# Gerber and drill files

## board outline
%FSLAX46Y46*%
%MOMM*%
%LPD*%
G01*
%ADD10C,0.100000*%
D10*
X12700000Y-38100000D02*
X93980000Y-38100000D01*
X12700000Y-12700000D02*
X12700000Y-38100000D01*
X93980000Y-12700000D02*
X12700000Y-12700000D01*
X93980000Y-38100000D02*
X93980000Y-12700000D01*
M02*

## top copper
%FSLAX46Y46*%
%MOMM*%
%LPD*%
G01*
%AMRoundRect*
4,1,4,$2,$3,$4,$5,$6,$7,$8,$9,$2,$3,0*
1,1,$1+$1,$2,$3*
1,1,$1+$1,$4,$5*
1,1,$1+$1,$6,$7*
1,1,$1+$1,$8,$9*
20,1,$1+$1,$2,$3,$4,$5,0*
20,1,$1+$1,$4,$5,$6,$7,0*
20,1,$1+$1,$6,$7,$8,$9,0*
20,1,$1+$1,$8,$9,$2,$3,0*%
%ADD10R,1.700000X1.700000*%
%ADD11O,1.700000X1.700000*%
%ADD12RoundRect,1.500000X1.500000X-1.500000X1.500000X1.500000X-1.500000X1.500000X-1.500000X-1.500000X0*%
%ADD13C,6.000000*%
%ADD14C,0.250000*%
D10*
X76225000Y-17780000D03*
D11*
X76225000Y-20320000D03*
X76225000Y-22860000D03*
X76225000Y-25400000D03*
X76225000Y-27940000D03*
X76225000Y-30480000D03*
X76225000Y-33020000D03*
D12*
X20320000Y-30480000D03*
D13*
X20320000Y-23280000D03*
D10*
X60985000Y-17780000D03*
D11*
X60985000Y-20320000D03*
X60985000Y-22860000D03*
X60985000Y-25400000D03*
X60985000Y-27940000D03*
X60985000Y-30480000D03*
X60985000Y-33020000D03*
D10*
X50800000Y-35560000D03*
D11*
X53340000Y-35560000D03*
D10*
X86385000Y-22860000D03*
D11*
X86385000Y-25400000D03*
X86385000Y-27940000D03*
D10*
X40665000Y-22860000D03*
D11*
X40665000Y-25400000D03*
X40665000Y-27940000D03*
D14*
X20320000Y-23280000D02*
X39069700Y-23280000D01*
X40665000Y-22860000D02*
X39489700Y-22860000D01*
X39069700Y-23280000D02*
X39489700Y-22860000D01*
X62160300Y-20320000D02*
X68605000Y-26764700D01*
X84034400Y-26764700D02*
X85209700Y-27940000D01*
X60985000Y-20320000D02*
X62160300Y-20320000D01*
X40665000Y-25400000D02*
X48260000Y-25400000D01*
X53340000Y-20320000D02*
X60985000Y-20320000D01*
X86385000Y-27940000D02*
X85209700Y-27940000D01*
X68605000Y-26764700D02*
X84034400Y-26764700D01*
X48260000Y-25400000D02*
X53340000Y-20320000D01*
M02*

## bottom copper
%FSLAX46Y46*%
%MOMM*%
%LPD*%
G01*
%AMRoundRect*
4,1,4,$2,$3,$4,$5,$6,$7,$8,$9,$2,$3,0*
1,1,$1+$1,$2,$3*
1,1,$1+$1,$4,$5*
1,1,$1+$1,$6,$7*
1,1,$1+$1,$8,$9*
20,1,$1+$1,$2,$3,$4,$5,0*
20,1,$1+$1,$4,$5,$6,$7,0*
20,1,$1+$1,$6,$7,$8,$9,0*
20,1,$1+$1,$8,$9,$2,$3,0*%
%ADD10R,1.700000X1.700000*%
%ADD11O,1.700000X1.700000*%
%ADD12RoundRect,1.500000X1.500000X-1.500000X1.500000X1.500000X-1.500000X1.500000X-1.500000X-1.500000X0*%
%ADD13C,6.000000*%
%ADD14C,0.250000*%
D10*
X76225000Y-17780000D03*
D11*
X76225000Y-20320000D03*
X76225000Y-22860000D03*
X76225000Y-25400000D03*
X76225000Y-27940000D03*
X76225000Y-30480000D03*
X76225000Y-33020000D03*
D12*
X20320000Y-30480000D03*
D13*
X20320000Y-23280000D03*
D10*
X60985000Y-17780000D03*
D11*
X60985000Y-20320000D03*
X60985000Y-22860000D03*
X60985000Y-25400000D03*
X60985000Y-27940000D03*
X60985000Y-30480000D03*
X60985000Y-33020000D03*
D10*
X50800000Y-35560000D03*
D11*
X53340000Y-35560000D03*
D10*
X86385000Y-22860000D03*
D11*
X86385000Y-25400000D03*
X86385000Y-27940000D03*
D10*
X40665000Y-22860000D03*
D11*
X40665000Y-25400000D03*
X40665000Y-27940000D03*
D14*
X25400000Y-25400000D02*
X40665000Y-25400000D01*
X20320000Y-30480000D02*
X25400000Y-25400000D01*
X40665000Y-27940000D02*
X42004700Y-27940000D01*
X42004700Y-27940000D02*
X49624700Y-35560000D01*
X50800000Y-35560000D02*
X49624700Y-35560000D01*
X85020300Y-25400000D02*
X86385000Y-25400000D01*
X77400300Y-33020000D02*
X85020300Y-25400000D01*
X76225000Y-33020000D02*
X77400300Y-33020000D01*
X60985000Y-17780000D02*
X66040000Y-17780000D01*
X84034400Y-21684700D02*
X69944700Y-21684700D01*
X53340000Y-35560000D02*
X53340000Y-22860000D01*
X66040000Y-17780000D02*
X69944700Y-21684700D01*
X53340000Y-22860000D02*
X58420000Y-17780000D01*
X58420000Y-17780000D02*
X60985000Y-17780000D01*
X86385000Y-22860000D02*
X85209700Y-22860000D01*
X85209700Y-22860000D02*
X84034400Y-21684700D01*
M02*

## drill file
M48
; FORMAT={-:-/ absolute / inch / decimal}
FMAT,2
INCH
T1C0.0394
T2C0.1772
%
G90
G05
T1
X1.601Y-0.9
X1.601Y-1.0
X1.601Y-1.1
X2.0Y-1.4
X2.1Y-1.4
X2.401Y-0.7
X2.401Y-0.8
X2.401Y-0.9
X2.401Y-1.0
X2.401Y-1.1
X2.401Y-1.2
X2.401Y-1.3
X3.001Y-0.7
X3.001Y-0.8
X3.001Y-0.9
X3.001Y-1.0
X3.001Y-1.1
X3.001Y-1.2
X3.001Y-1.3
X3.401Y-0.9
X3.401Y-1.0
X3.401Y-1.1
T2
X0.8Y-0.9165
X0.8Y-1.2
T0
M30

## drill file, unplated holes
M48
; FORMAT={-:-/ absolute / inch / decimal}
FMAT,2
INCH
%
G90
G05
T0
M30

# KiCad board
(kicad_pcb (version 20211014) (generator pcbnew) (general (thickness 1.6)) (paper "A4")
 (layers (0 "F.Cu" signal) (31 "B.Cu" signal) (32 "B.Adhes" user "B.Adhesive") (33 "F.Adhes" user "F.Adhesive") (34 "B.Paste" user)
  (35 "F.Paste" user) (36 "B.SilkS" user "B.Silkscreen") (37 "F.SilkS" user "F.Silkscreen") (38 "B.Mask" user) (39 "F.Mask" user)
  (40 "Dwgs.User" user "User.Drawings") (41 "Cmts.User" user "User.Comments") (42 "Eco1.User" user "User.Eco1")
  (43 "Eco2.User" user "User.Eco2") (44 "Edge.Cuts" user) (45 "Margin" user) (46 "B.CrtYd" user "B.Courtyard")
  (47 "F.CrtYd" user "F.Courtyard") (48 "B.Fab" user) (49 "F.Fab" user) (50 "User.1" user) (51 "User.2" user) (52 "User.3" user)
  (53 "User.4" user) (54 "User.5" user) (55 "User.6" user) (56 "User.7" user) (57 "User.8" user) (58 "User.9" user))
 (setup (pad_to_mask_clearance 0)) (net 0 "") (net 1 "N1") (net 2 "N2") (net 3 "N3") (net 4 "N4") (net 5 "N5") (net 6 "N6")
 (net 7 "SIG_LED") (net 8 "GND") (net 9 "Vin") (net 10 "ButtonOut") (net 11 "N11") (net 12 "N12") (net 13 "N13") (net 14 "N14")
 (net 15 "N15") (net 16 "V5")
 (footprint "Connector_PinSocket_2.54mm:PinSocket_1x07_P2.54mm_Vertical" (layer "F.Cu") (at 76.225 17.78)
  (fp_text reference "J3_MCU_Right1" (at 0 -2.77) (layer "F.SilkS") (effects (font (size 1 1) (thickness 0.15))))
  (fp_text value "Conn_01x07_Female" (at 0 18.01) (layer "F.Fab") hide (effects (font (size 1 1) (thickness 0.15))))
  (pad "1" thru_hole rect (at 0 0) (size 1.7 1.7) (drill 1) (layers *.Cu *.Mask) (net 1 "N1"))
  (pad "2" thru_hole oval (at 0 2.54) (size 1.7 1.7) (drill 1) (layers *.Cu *.Mask) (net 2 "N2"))
  (pad "3" thru_hole oval (at 0 5.08) (size 1.7 1.7) (drill 1) (layers *.Cu *.Mask) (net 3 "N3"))
  (pad "4" thru_hole oval (at 0 7.62) (size 1.7 1.7) (drill 1) (layers *.Cu *.Mask) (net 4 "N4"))
  (pad "5" thru_hole oval (at 0 10.16) (size 1.7 1.7) (drill 1) (layers *.Cu *.Mask) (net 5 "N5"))
  (pad "6" thru_hole oval (at 0 12.7) (size 1.7 1.7) (drill 1) (layers *.Cu *.Mask) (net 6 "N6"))
  (pad "7" thru_hole oval (at 0 15.24) (size 1.7 1.7) (drill 1) (layers *.Cu *.Mask) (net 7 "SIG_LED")))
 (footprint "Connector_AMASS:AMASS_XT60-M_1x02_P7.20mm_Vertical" (layer "F.Cu") (at 20.32 30.48 90)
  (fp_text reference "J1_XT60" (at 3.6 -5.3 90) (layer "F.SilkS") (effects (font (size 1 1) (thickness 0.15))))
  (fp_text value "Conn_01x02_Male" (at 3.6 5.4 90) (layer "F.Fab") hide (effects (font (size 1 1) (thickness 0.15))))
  (pad "1" thru_hole roundrect (at 0 0 90) (size 6 6) (drill 4.5) (layers *.Cu *.Mask) (roundrect_rratio 0.25) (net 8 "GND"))
  (pad "2" thru_hole circle (at 7.2 0 90) (size 6 6) (drill 4.5) (layers *.Cu *.Mask) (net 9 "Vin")))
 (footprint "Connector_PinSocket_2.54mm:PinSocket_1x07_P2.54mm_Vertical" (layer "F.Cu") (at 60.985 17.78)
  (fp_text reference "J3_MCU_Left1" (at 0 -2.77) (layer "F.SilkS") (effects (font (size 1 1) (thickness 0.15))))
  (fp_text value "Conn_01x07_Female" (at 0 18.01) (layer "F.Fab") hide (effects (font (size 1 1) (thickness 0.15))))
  (pad "1" thru_hole rect (at 0 0) (size 1.7 1.7) (drill 1) (layers *.Cu *.Mask) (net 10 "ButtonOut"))
  (pad "2" thru_hole oval (at 0 2.54) (size 1.7 1.7) (drill 1) (layers *.Cu *.Mask) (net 8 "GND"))
  (pad "3" thru_hole oval (at 0 5.08) (size 1.7 1.7) (drill 1) (layers *.Cu *.Mask) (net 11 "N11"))
  (pad "4" thru_hole oval (at 0 7.62) (size 1.7 1.7) (drill 1) (layers *.Cu *.Mask) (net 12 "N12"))
  (pad "5" thru_hole oval (at 0 10.16) (size 1.7 1.7) (drill 1) (layers *.Cu *.Mask) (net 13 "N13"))
  (pad "6" thru_hole oval (at 0 12.7) (size 1.7 1.7) (drill 1) (layers *.Cu *.Mask) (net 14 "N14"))
  (pad "7" thru_hole oval (at 0 15.24) (size 1.7 1.7) (drill 1) (layers *.Cu *.Mask) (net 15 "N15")))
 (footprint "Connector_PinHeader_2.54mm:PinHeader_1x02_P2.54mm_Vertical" (layer "F.Cu") (at 50.8 35.56 90)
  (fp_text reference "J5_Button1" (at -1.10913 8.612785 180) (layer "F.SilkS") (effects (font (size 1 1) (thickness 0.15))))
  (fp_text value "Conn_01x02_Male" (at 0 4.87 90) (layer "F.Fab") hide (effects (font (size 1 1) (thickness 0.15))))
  (pad "1" thru_hole rect (at 0 0 90) (size 1.7 1.7) (drill 1) (layers *.Cu *.Mask) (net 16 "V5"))
  (pad "2" thru_hole oval (at 0 2.54 90) (size 1.7 1.7) (drill 1) (layers *.Cu *.Mask) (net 10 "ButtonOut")))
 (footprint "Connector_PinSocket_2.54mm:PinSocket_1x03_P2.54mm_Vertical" (layer "F.Cu") (at 86.385 22.86)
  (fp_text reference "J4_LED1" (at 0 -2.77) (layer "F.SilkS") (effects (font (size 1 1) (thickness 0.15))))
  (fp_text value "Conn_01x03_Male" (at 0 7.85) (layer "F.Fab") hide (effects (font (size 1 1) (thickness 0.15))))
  (pad "1" thru_hole rect (at 0 0) (size 1.7 1.7) (drill 1) (layers *.Cu *.Mask) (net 10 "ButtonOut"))
  (pad "2" thru_hole oval (at 0 2.54) (size 1.7 1.7) (drill 1) (layers *.Cu *.Mask) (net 7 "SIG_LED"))
  (pad "3" thru_hole oval (at 0 5.08) (size 1.7 1.7) (drill 1) (layers *.Cu *.Mask) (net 8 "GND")))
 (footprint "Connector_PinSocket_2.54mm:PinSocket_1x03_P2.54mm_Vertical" (layer "F.Cu") (at 40.665 22.86)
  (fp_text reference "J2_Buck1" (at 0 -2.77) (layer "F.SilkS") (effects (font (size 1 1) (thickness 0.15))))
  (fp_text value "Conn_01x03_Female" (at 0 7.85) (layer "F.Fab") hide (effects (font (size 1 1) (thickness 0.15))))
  (pad "1" thru_hole rect (at 0 0) (size 1.7 1.7) (drill 1) (layers *.Cu *.Mask) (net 9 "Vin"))
  (pad "2" thru_hole oval (at 0 2.54) (size 1.7 1.7) (drill 1) (layers *.Cu *.Mask) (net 8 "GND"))
  (pad "3" thru_hole oval (at 0 5.08) (size 1.7 1.7) (drill 1) (layers *.Cu *.Mask) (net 16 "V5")))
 (gr_line (start 12.7 38.1) (end 93.98 38.1) (layer "Edge.Cuts") (width 0.1))
 (gr_line (start 12.7 12.7) (end 12.7 38.1) (layer "Edge.Cuts") (width 0.1))
 (gr_line (start 93.98 12.7) (end 12.7 12.7) (layer "Edge.Cuts") (width 0.1))
 (gr_line (start 93.98 38.1) (end 93.98 12.7) (layer "Edge.Cuts") (width 0.1))
 (segment (start 20.32 23.28) (end 39.0697 23.28) (width 0.25) (layer "F.Cu") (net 9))
 (segment (start 40.665 22.86) (end 39.4897 22.86) (width 0.25) (layer "F.Cu") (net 9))
 (segment (start 39.0697 23.28) (end 39.4897 22.86) (width 0.25) (layer "F.Cu") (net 9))
 (segment (start 62.1603 20.32) (end 68.605 26.7647) (width 0.25) (layer "F.Cu") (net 8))
 (segment (start 84.0344 26.7647) (end 85.2097 27.94) (width 0.25) (layer "F.Cu") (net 8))
 (segment (start 60.985 20.32) (end 62.1603 20.32) (width 0.25) (layer "F.Cu") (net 8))
 (segment (start 40.665 25.4) (end 48.26 25.4) (width 0.25) (layer "F.Cu") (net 8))
 (segment (start 53.34 20.32) (end 60.985 20.32) (width 0.25) (layer "F.Cu") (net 8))
 (segment (start 86.385 27.94) (end 85.2097 27.94) (width 0.25) (layer "F.Cu") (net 8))
 (segment (start 68.605 26.7647) (end 84.0344 26.7647) (width 0.25) (layer "F.Cu") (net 8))
 (segment (start 48.26 25.4) (end 53.34 20.32) (width 0.25) (layer "F.Cu") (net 8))
 (segment (start 25.4 25.4) (end 40.665 25.4) (width 0.25) (layer "B.Cu") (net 8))
 (segment (start 20.32 30.48) (end 25.4 25.4) (width 0.25) (layer "B.Cu") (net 8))
 (segment (start 40.665 27.94) (end 42.0047 27.94) (width 0.25) (layer "B.Cu") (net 16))
 (segment (start 42.0047 27.94) (end 49.6247 35.56) (width 0.25) (layer "B.Cu") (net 16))
 (segment (start 50.8 35.56) (end 49.6247 35.56) (width 0.25) (layer "B.Cu") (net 16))
 (segment (start 85.0203 25.4) (end 86.385 25.4) (width 0.25) (layer "B.Cu") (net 7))
 (segment (start 77.4003 33.02) (end 85.0203 25.4) (width 0.25) (layer "B.Cu") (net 7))
 (segment (start 76.225 33.02) (end 77.4003 33.02) (width 0.25) (layer "B.Cu") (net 7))
 (segment (start 60.985 17.78) (end 66.04 17.78) (width 0.25) (layer "B.Cu") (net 10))
 (segment (start 84.0344 21.6847) (end 69.9447 21.6847) (width 0.25) (layer "B.Cu") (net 10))
 (segment (start 53.34 35.56) (end 53.34 22.86) (width 0.25) (layer "B.Cu") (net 10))
 (segment (start 66.04 17.78) (end 69.9447 21.6847) (width 0.25) (layer "B.Cu") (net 10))
 (segment (start 53.34 22.86) (end 58.42 17.78) (width 0.25) (layer "B.Cu") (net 10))
 (segment (start 58.42 17.78) (end 60.985 17.78) (width 0.25) (layer "B.Cu") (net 10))
 (segment (start 86.385 22.86) (end 85.2097 22.86) (width 0.25) (layer "B.Cu") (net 10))
 (segment (start 85.2097 22.86) (end 84.0344 21.6847) (width 0.25) (layer "B.Cu") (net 10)))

